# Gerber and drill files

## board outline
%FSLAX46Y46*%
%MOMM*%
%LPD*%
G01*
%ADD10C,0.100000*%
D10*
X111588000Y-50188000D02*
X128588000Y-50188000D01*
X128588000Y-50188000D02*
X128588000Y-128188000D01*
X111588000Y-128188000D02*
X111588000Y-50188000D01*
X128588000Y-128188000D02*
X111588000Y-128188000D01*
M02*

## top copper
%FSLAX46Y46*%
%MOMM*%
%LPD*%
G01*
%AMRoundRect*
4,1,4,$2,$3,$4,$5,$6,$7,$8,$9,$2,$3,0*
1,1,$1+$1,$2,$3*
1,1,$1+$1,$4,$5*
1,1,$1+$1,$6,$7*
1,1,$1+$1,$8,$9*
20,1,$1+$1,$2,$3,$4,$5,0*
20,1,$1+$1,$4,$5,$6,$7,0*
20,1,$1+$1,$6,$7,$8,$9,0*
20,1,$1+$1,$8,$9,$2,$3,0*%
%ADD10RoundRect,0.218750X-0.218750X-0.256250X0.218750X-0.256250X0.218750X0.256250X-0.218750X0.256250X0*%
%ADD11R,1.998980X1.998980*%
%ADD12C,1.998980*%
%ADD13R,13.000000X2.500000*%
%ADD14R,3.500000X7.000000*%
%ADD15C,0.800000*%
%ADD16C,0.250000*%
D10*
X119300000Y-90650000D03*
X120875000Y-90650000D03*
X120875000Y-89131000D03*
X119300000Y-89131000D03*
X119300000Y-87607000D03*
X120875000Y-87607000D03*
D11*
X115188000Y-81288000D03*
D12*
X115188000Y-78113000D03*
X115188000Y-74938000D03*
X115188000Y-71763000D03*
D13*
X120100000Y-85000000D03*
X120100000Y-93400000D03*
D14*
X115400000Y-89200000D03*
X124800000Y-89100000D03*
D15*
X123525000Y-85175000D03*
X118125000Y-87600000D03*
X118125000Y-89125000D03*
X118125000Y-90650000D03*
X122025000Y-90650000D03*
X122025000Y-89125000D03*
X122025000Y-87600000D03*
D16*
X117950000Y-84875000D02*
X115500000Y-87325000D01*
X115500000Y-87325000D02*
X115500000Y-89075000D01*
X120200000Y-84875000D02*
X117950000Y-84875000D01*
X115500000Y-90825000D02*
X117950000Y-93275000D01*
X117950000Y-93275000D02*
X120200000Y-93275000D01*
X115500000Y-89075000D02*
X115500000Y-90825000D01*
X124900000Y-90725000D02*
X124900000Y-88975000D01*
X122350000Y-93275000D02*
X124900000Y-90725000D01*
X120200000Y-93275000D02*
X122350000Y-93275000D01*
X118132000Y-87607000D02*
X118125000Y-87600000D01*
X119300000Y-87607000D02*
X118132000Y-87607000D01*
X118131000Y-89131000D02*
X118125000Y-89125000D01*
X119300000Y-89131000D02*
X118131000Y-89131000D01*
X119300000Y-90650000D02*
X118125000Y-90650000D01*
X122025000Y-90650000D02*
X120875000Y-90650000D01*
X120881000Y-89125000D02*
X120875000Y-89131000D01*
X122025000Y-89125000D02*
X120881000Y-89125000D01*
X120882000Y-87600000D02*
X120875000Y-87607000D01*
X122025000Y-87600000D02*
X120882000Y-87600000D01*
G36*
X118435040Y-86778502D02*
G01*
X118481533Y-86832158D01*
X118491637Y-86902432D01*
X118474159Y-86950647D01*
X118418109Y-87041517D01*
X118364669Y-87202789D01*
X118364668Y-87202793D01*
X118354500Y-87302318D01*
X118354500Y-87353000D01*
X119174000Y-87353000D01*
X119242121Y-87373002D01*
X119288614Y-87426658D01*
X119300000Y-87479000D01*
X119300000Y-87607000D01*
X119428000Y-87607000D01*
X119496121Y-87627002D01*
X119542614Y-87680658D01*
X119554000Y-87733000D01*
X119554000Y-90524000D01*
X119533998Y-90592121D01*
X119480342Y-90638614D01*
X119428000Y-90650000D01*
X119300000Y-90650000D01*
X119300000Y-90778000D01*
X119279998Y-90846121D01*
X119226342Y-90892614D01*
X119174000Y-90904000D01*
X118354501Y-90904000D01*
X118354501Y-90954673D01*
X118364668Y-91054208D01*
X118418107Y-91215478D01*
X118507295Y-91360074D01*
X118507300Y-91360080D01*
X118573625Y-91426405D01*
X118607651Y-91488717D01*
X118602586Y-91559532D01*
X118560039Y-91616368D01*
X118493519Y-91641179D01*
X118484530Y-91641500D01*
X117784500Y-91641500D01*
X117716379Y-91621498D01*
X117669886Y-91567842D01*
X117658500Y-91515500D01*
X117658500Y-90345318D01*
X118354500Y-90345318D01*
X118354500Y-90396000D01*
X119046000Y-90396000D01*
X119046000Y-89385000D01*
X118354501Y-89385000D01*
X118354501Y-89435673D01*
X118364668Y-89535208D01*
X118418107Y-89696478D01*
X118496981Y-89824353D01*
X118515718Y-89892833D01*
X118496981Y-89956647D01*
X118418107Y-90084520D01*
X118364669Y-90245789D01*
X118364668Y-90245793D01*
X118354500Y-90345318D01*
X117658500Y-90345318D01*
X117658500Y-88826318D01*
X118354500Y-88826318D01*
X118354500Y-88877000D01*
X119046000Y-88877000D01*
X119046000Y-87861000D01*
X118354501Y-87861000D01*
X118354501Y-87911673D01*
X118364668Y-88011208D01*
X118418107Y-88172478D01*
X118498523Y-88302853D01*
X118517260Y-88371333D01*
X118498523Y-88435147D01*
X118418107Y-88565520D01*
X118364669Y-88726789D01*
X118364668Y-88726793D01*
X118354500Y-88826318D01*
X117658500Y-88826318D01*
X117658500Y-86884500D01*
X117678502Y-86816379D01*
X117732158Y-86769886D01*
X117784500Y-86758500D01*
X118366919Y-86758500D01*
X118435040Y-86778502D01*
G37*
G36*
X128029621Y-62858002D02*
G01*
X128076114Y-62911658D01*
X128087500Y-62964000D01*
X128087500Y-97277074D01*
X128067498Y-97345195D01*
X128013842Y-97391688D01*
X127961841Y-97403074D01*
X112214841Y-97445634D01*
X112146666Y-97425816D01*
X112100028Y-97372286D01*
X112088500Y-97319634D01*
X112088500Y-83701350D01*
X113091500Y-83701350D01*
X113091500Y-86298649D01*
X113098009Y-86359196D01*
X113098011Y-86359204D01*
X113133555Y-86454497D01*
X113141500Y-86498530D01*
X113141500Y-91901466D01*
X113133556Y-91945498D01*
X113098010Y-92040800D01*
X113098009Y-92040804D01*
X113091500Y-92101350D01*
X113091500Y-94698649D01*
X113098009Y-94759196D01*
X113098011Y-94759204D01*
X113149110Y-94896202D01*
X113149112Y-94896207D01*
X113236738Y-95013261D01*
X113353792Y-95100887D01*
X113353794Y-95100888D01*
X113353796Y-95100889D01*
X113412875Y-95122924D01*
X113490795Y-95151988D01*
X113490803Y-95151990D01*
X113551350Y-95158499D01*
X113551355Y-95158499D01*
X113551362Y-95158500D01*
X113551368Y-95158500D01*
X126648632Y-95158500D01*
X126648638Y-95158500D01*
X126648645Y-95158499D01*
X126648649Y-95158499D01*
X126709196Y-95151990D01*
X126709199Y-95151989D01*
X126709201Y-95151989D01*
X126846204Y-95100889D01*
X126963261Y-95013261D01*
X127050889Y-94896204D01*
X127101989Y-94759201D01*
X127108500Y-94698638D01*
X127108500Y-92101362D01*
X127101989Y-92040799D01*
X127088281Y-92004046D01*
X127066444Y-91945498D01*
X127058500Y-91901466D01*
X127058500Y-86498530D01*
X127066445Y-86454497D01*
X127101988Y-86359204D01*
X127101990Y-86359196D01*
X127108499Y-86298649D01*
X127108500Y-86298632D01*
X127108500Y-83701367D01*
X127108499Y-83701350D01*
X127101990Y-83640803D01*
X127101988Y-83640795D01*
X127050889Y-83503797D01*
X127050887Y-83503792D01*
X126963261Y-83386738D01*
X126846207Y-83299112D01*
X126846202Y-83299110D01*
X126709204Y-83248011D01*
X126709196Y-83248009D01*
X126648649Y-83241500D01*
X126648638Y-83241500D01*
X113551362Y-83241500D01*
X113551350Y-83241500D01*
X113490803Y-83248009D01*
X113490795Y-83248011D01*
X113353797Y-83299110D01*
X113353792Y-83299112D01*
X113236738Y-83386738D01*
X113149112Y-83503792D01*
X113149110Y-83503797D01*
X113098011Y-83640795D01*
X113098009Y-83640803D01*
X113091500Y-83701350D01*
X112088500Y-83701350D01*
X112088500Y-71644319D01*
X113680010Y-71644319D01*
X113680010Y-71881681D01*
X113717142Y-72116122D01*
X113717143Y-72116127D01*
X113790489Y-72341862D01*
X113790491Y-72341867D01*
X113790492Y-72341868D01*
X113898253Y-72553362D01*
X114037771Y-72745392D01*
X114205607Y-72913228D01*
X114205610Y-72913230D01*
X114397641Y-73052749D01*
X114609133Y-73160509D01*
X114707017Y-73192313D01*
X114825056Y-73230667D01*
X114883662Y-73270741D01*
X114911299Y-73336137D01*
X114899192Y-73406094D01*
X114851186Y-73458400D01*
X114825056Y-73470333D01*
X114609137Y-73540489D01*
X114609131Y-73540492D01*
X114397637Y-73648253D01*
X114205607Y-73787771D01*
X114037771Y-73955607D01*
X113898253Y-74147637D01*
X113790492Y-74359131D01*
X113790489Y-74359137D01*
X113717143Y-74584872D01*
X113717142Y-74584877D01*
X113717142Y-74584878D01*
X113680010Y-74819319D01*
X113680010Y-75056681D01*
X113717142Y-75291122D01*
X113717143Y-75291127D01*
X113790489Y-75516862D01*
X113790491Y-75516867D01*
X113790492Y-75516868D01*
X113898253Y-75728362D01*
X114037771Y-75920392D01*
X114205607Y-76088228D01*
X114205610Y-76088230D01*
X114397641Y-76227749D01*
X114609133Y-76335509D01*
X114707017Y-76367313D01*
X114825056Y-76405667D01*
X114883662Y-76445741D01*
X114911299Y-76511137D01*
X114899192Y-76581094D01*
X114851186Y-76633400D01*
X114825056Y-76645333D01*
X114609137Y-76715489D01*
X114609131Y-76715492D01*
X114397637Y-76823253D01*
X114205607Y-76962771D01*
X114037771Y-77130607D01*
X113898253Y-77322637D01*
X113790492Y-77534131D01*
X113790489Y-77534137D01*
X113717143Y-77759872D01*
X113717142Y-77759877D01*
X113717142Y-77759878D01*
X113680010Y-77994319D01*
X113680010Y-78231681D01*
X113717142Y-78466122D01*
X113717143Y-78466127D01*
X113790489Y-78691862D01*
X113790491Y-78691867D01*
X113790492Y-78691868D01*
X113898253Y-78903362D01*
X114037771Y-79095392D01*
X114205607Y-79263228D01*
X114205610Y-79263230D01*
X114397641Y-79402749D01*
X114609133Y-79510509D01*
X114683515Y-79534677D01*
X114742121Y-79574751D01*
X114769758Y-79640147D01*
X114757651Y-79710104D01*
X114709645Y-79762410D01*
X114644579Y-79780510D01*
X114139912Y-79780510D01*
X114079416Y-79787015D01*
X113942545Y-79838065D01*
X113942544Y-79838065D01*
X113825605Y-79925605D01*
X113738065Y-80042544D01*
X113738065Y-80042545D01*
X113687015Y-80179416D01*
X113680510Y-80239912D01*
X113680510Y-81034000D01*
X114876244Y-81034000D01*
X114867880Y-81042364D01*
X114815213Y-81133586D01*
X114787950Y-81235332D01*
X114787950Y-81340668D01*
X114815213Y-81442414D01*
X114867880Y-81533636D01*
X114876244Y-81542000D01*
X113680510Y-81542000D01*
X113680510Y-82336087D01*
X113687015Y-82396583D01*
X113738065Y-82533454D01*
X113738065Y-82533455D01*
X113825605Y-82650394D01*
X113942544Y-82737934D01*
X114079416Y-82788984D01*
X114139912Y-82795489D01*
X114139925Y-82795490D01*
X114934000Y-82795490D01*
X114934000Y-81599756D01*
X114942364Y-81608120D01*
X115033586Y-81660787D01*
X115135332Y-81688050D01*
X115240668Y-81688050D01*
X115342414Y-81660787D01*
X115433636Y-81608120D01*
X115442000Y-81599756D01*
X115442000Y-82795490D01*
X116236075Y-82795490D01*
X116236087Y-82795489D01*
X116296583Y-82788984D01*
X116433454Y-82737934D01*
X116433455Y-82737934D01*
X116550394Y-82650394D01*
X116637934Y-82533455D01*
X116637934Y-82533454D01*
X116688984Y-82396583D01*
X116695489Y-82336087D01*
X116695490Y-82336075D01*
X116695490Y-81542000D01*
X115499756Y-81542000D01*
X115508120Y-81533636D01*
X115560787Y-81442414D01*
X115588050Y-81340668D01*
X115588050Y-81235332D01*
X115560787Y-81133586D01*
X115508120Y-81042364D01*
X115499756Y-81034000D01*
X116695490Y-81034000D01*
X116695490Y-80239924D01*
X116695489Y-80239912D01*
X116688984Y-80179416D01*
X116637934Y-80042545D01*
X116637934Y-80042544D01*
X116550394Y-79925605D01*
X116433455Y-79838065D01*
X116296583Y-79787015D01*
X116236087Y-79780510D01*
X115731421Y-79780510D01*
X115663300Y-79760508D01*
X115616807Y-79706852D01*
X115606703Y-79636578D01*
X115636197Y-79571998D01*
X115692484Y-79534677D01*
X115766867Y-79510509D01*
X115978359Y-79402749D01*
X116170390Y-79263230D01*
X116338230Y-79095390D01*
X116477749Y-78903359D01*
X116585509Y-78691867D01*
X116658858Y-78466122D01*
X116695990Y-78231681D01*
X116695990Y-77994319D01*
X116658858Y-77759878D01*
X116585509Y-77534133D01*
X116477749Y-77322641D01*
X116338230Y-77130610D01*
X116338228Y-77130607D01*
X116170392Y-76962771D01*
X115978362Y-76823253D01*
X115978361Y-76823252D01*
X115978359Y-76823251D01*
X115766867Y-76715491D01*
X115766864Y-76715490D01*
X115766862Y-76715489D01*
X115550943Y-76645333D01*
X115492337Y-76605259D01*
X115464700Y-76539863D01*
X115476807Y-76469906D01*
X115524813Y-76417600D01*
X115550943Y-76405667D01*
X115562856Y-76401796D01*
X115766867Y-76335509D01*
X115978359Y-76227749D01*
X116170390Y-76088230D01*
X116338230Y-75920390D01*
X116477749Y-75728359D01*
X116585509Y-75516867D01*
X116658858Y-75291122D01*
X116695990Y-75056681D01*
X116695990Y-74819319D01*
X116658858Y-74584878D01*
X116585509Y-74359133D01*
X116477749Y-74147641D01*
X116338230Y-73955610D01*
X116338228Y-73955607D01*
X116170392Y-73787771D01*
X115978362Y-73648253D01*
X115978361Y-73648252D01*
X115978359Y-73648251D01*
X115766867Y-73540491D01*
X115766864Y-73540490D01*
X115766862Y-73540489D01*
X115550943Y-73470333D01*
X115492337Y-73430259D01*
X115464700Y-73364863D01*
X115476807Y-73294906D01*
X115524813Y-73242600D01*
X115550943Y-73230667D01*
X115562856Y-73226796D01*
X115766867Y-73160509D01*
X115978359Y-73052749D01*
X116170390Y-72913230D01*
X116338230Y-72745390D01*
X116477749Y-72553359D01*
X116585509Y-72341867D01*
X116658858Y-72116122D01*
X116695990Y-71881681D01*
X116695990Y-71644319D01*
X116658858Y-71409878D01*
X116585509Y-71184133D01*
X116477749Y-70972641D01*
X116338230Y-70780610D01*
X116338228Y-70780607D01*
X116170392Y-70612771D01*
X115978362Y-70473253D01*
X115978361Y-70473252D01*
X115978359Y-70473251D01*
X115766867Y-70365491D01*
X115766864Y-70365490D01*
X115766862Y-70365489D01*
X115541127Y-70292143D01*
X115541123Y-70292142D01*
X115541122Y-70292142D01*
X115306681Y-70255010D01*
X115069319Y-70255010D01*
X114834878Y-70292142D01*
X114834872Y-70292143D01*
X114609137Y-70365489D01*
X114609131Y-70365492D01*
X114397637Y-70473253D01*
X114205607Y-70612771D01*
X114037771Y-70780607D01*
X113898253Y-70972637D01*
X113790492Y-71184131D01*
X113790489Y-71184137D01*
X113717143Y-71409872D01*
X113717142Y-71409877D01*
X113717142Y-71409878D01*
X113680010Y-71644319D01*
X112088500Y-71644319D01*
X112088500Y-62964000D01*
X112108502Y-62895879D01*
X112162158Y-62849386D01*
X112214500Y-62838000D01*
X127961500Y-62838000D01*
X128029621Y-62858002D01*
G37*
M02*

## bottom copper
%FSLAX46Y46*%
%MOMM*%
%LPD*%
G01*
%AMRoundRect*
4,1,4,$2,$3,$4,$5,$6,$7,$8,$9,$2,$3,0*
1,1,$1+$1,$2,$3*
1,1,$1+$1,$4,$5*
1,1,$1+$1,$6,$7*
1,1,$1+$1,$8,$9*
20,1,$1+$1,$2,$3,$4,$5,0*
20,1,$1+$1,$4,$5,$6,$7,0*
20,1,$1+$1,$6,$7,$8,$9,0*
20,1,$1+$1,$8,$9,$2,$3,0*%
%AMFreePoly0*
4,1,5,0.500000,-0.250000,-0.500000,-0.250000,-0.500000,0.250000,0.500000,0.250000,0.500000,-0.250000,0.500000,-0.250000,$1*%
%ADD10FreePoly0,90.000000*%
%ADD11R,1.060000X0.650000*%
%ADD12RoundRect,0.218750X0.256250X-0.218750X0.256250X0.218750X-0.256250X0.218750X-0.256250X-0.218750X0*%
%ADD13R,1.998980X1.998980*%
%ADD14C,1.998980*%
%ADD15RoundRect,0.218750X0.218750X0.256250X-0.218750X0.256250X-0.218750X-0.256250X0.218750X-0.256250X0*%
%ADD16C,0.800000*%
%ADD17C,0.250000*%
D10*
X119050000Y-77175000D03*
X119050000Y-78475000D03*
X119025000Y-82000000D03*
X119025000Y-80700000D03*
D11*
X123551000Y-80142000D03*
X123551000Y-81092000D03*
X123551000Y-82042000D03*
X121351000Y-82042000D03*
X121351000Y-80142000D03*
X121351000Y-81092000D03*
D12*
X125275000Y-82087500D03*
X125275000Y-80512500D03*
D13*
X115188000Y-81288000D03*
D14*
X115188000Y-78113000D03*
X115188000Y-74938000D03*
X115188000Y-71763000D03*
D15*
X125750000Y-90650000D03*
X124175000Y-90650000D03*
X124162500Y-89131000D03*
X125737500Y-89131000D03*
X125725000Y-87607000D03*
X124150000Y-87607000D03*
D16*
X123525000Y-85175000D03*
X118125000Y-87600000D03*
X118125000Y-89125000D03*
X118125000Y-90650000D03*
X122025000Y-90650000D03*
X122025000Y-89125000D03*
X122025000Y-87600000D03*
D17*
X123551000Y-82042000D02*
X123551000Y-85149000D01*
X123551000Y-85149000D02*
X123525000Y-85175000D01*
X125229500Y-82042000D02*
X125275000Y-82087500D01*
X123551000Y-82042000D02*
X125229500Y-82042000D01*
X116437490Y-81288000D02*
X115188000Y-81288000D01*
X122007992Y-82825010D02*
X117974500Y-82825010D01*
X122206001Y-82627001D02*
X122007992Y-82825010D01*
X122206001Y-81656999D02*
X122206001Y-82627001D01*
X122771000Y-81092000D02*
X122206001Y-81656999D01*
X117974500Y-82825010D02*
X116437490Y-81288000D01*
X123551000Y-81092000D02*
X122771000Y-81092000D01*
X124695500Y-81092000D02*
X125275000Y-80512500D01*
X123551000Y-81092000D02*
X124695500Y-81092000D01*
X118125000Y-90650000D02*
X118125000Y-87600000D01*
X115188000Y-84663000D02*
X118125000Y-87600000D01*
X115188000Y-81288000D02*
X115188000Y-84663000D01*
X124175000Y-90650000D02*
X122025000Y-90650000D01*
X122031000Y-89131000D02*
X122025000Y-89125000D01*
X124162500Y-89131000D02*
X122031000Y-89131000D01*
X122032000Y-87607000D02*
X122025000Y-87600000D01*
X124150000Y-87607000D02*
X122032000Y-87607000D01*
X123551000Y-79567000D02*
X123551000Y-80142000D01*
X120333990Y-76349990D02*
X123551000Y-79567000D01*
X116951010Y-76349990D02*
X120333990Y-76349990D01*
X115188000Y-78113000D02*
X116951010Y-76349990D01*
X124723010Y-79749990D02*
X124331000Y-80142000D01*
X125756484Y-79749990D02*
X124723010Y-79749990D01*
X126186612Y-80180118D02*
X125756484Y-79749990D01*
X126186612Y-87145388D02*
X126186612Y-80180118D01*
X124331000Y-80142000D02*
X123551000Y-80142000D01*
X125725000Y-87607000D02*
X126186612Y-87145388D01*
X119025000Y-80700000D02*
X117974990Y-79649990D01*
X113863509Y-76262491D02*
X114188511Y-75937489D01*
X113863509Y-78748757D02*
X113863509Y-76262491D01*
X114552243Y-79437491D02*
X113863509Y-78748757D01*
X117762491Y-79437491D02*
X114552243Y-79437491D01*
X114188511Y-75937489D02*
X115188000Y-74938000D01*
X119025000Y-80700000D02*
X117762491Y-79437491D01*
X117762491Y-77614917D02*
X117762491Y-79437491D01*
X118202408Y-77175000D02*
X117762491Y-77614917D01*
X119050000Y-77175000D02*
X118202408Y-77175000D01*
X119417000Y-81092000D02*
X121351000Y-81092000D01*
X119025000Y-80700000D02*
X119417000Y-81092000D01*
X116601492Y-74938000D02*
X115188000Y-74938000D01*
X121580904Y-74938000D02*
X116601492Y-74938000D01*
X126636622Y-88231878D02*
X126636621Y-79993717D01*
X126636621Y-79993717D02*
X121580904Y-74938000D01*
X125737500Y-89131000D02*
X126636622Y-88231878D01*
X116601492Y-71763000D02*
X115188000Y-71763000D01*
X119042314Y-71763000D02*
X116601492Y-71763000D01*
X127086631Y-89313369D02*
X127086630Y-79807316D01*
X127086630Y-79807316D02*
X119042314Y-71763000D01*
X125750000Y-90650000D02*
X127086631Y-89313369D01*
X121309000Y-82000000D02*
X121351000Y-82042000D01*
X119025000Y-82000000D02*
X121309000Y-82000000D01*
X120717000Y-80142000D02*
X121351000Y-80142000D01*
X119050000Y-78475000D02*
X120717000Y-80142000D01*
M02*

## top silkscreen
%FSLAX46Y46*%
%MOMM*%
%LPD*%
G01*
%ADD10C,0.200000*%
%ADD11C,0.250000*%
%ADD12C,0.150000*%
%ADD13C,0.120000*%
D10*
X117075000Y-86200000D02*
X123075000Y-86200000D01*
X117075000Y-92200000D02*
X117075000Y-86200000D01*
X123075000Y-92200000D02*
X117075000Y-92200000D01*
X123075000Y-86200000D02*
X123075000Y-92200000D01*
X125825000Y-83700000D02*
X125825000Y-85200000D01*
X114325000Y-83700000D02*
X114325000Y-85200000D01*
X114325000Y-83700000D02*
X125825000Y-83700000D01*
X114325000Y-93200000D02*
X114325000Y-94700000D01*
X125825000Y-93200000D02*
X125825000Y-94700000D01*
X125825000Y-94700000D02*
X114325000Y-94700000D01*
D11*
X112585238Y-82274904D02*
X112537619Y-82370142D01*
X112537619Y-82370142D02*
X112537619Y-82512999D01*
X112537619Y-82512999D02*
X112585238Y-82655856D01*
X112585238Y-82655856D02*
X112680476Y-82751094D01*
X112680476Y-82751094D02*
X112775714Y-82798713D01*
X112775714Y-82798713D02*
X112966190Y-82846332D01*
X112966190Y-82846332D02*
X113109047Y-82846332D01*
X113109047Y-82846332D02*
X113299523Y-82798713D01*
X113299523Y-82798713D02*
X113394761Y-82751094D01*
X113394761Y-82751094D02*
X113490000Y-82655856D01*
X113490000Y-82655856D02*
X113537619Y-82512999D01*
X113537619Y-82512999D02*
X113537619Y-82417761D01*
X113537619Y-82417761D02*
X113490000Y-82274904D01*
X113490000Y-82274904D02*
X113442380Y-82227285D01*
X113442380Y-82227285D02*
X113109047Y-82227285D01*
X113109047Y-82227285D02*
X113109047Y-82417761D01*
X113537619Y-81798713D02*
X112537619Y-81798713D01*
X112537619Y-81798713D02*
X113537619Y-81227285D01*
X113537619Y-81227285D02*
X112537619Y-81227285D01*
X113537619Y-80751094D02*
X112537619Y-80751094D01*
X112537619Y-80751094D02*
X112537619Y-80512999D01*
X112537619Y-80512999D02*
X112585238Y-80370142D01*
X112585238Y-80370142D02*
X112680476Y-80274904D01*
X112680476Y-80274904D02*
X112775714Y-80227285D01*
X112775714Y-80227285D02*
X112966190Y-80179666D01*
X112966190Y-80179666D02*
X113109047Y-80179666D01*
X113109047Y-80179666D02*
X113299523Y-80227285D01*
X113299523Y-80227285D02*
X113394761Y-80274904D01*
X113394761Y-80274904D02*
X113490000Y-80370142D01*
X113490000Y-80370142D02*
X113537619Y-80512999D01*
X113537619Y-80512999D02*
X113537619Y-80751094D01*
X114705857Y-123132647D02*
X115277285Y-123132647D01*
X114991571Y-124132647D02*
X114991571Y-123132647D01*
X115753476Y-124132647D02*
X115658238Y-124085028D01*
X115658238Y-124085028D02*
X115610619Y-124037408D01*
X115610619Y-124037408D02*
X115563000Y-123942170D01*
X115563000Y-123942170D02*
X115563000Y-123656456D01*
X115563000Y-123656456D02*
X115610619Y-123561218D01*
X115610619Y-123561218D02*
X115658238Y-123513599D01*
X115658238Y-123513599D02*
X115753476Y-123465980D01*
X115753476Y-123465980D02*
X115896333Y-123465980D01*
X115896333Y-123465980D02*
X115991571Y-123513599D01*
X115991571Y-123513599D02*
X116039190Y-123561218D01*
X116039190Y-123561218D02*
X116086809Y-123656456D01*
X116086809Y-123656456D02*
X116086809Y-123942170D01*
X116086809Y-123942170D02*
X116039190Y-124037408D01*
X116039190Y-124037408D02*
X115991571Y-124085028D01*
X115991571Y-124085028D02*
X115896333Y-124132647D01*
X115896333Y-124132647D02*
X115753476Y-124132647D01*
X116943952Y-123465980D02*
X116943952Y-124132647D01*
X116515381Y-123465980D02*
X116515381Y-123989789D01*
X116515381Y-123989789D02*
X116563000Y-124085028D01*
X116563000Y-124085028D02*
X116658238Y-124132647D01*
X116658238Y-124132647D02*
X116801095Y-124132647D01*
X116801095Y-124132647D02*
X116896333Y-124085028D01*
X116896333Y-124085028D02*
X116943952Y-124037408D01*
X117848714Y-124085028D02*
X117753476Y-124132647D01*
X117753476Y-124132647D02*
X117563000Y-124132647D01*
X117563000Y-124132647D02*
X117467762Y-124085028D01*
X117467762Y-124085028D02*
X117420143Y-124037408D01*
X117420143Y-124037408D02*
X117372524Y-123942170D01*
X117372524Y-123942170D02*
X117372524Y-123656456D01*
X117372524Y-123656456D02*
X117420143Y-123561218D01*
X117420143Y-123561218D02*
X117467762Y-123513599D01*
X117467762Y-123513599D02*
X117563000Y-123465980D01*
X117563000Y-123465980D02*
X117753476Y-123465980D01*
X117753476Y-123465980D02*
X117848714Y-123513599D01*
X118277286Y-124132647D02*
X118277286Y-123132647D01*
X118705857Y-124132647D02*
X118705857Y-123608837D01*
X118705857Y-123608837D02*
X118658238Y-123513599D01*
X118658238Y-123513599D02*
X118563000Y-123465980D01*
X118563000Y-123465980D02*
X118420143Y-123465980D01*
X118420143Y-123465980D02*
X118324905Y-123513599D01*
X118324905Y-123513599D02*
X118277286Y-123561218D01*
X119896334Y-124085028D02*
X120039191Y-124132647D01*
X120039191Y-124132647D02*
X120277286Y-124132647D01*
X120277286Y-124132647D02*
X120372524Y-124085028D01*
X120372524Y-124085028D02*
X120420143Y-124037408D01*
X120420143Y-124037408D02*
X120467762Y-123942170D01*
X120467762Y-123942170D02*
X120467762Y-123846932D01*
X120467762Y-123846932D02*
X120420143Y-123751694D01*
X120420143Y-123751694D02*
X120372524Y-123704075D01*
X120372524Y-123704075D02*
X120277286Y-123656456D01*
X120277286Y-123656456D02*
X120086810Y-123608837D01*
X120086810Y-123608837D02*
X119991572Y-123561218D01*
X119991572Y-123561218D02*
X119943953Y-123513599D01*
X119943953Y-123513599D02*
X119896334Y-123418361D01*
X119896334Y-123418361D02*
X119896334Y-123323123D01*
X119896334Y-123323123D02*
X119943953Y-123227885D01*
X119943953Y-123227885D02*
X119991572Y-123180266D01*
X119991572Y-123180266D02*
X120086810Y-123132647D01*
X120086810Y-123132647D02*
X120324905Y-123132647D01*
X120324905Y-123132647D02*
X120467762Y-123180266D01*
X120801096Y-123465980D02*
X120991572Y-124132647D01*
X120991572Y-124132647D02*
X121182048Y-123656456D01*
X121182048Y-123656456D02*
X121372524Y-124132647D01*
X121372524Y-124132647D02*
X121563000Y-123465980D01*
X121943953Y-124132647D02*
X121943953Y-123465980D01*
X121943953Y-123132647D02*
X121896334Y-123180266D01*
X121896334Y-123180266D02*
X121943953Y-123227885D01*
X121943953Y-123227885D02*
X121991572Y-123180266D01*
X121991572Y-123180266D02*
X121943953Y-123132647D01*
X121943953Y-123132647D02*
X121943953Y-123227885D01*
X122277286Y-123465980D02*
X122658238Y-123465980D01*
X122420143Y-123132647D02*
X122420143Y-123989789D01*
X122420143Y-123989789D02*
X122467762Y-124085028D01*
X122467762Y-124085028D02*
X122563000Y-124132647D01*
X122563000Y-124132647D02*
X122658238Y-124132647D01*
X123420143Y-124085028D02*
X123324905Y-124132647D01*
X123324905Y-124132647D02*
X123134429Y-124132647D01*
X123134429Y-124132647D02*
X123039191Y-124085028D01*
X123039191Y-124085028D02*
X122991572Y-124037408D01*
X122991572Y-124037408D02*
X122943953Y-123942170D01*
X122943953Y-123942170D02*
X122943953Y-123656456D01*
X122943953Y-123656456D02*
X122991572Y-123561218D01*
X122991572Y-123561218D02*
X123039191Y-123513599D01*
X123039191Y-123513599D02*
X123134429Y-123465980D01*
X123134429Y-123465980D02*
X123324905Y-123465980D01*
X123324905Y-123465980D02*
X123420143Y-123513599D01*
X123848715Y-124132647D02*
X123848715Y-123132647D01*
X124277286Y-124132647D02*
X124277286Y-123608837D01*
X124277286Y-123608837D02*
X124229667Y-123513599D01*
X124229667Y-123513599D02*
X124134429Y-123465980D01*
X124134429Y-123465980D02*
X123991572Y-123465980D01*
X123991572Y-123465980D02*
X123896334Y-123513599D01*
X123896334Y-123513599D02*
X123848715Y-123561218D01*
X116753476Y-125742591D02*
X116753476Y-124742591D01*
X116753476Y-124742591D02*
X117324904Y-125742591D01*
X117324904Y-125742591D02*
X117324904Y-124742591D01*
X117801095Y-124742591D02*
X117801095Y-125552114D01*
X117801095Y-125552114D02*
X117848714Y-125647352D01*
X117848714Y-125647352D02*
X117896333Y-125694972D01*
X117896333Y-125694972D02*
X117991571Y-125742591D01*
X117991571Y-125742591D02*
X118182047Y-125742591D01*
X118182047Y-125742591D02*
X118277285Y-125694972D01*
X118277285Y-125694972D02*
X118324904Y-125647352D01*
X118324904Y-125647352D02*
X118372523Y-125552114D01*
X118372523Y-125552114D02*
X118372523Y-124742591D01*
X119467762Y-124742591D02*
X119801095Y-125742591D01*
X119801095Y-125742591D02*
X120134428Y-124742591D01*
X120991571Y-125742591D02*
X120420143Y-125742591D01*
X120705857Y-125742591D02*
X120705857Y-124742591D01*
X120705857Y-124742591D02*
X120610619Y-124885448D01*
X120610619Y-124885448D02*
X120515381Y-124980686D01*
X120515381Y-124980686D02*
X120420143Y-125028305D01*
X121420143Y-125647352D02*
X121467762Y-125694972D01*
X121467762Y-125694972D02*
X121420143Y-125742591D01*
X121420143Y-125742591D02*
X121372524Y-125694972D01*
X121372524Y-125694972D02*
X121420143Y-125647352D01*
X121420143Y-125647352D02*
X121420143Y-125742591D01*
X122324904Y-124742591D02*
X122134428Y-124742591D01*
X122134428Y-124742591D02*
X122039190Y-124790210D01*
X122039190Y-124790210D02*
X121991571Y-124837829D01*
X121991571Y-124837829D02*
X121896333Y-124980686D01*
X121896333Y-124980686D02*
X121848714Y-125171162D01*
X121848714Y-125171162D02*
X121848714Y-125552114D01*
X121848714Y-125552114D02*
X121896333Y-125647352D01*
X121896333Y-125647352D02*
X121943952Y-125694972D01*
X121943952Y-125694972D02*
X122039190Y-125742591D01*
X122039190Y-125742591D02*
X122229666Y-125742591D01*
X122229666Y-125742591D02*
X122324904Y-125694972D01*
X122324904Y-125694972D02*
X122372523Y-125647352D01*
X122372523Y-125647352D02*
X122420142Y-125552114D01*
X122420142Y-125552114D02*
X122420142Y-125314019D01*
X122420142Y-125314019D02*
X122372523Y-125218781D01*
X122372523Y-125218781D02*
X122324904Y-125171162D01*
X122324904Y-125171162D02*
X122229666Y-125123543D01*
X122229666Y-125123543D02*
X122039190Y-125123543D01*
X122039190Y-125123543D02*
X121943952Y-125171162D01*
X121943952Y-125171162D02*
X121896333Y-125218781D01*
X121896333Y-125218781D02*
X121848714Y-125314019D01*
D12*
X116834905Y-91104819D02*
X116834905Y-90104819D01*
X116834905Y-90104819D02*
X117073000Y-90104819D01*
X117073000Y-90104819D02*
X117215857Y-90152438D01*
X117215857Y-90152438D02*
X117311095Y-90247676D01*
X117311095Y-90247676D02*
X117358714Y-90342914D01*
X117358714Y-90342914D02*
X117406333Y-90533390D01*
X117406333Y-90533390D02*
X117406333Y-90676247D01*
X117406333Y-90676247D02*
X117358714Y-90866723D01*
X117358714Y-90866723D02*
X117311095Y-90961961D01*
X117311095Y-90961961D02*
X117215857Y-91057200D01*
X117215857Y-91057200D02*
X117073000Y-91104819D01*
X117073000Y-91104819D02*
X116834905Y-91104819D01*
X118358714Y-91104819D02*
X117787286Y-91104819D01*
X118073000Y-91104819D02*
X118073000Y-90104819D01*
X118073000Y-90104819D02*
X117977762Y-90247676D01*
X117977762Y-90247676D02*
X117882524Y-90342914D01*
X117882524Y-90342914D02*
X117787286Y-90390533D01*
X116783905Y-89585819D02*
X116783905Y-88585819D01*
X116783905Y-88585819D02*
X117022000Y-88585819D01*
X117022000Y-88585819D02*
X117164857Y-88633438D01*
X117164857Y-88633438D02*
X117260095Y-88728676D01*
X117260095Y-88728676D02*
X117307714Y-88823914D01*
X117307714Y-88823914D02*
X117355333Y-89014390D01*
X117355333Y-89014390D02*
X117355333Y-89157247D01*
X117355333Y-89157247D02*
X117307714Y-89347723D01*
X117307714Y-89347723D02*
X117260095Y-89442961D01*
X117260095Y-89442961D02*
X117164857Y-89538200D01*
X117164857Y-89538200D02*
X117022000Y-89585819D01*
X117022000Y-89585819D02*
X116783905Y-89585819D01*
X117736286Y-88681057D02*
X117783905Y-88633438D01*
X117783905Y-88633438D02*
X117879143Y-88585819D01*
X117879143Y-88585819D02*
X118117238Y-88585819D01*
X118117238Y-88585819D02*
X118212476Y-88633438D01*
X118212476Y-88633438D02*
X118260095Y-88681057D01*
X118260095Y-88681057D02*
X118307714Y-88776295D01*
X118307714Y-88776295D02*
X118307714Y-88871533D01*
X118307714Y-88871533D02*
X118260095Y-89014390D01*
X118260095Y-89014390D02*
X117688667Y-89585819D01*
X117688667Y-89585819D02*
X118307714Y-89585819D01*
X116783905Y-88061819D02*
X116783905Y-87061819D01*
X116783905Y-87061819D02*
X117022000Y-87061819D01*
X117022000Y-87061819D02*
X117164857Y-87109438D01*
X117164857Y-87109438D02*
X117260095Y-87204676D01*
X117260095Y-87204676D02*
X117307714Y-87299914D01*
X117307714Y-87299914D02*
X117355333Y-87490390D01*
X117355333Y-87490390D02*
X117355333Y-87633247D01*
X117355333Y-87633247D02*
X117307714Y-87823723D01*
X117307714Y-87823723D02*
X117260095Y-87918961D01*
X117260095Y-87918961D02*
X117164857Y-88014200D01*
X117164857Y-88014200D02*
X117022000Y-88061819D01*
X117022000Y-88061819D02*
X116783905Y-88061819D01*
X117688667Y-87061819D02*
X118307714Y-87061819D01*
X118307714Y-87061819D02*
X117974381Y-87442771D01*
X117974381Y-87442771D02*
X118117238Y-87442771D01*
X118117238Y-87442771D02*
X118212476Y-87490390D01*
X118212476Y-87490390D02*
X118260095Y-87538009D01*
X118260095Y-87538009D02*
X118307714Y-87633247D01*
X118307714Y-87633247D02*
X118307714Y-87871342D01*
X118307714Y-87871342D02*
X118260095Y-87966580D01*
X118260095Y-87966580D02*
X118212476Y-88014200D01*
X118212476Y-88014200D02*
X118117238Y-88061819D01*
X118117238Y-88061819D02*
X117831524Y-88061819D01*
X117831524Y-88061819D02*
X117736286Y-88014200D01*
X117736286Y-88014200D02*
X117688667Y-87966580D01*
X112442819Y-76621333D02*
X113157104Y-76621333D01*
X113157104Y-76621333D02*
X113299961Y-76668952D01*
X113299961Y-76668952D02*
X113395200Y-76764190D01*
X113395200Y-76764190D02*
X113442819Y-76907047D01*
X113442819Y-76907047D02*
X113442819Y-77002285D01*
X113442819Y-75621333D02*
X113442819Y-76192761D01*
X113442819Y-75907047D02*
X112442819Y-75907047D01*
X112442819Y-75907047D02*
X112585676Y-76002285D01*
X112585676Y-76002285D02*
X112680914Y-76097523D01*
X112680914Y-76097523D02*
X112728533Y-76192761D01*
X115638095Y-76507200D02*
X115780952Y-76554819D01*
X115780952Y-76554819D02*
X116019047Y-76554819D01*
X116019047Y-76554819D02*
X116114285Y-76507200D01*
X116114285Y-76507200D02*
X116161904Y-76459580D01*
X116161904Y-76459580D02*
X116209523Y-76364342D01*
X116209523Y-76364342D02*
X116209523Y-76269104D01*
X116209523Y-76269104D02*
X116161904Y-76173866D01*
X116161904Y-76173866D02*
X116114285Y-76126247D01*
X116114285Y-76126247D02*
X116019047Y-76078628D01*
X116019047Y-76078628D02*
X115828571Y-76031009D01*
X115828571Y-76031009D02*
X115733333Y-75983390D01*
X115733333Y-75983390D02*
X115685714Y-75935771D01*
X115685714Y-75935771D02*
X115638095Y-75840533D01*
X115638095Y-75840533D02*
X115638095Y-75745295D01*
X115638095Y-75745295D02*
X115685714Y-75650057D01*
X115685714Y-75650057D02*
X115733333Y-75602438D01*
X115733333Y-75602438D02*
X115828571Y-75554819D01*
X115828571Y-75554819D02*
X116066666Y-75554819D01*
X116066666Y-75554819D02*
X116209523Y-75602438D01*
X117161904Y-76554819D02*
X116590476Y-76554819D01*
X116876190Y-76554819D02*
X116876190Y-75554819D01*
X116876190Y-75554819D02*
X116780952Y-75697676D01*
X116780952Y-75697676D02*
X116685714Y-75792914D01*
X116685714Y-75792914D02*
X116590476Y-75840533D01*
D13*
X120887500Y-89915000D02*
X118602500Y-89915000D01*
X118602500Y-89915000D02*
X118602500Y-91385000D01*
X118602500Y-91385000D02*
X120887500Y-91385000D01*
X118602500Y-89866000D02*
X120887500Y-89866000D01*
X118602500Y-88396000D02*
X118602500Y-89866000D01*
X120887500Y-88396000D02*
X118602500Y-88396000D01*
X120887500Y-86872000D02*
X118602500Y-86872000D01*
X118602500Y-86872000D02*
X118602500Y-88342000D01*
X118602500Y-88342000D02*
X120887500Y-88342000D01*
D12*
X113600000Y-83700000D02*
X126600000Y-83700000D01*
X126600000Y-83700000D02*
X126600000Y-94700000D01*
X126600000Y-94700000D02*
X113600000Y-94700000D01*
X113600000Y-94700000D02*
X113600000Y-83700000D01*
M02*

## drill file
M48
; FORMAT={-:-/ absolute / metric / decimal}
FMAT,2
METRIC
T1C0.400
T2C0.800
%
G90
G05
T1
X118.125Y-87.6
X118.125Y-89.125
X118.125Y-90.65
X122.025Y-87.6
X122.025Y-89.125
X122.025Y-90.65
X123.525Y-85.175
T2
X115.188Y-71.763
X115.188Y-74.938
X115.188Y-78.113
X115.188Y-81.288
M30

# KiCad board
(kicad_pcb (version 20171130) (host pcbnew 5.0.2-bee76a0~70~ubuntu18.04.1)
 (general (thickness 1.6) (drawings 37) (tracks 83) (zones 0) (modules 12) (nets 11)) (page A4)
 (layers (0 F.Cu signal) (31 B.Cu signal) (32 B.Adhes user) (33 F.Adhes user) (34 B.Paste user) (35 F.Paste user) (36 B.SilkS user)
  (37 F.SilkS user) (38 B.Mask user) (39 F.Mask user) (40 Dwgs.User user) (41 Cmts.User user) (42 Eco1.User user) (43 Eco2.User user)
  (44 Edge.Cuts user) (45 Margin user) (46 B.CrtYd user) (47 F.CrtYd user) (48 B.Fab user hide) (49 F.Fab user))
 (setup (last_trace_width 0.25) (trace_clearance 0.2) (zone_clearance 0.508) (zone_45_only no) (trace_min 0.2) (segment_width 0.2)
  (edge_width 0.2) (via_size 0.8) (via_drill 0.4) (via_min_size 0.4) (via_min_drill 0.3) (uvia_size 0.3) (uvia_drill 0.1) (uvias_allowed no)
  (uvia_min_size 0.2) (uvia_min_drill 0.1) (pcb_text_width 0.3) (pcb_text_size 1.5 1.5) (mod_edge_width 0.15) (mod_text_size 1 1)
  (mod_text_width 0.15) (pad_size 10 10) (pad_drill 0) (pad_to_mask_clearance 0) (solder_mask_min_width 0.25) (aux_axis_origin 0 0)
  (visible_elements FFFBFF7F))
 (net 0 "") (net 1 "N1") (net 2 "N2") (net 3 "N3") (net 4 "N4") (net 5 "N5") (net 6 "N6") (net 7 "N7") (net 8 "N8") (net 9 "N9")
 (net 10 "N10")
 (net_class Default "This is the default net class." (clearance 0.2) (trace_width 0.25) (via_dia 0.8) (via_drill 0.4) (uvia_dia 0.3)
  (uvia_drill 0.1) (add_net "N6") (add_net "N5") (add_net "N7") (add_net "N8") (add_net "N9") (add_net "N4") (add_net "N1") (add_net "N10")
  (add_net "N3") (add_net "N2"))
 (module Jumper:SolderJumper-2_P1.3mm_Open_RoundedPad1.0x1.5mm (layer B.Cu) (at 119.05 77.825 90)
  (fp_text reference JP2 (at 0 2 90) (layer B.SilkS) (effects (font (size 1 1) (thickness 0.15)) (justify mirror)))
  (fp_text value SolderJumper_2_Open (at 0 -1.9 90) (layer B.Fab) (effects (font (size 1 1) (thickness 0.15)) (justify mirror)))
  (pad 2 smd custom (at 0.65 0 90) (size 1 0.5) (layers B.Cu B.Mask) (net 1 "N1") (zone_connect 0)
   (options (clearance outline) (anchor rect)) (primitives))
  (pad 1 smd custom (at -0.65 0 90) (size 1 0.5) (layers B.Cu B.Mask) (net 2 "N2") (zone_connect 0)
   (options (clearance outline) (anchor rect)) (primitives)))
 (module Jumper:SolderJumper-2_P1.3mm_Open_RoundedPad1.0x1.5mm (layer B.Cu) (at 119.025 81.35 90)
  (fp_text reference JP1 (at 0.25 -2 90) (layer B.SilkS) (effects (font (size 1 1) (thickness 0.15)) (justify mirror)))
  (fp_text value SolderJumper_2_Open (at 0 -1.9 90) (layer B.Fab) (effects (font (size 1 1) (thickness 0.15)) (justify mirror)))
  (pad 1 smd custom (at -0.65 0 90) (size 1 0.5) (layers B.Cu B.Mask) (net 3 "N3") (zone_connect 0)
   (options (clearance outline) (anchor rect)) (primitives))
  (pad 2 smd custom (at 0.65 0 90) (size 1 0.5) (layers B.Cu B.Mask) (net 1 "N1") (zone_connect 0)
   (options (clearance outline) (anchor rect)) (primitives)))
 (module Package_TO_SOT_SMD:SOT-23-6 (layer B.Cu) (at 122.451 81.092 180)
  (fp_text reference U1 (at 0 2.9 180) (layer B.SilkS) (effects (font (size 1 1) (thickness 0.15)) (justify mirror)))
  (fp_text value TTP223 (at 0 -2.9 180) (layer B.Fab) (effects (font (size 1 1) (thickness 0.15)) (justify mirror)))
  (pad 1 smd rect (at -1.1 0.95 180) (size 1.06 0.65) (layers B.Cu B.Paste B.Mask) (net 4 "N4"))
  (pad 2 smd rect (at -1.1 0 180) (size 1.06 0.65) (layers B.Cu B.Paste B.Mask) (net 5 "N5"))
  (pad 3 smd rect (at -1.1 -0.95 180) (size 1.06 0.65) (layers B.Cu B.Paste B.Mask) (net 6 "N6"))
  (pad 4 smd rect (at 1.1 -0.95 180) (size 1.06 0.65) (layers B.Cu B.Paste B.Mask) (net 3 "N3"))
  (pad 6 smd rect (at 1.1 0.95 180) (size 1.06 0.65) (layers B.Cu B.Paste B.Mask) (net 2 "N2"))
  (pad 5 smd rect (at 1.1 0 180) (size 1.06 0.65) (layers B.Cu B.Paste B.Mask) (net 1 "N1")))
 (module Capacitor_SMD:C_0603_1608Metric (layer B.Cu) (at 125.275 81.3 90)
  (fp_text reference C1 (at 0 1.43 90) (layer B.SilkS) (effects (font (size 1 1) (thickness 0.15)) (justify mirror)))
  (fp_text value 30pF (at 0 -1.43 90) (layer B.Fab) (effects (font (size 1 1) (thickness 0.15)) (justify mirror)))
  (pad 1 smd roundrect (at -0.7875 0 90) (size 0.875 0.95) (layers B.Cu B.Paste B.Mask) (roundrect_rratio 0.25) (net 6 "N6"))
  (pad 2 smd roundrect (at 0.7875 0 90) (size 0.875 0.95) (layers B.Cu B.Paste B.Mask) (roundrect_rratio 0.25) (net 5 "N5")))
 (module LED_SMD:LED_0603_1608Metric (layer F.Cu) (at 120.0875 90.65)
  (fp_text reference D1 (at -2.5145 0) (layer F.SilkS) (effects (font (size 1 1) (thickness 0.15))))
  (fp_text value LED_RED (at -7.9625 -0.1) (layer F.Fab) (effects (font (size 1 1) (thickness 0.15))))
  (fp_line (start 0.8 -0.735) (end -1.485 -0.735) (layer F.SilkS) (width 0.12))
  (fp_line (start -1.485 -0.735) (end -1.485 0.735) (layer F.SilkS) (width 0.12))
  (fp_line (start -1.485 0.735) (end 0.8 0.735) (layer F.SilkS) (width 0.12))
  (pad 1 smd roundrect (at -0.7875 0) (size 0.875 0.95) (layers F.Cu F.Paste F.Mask) (roundrect_rratio 0.25) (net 5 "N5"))
  (pad 2 smd roundrect (at 0.7875 0) (size 0.875 0.95) (layers F.Cu F.Paste F.Mask) (roundrect_rratio 0.25) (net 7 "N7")))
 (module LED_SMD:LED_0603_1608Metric (layer F.Cu) (at 120.0875 89.131)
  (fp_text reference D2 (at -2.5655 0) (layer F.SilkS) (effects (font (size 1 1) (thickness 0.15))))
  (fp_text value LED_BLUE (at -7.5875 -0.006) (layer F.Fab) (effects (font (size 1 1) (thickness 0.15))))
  (fp_line (start -1.485 0.735) (end 0.8 0.735) (layer F.SilkS) (width 0.12))
  (fp_line (start -1.485 -0.735) (end -1.485 0.735) (layer F.SilkS) (width 0.12))
  (fp_line (start 0.8 -0.735) (end -1.485 -0.735) (layer F.SilkS) (width 0.12))
  (pad 2 smd roundrect (at 0.7875 0) (size 0.875 0.95) (layers F.Cu F.Paste F.Mask) (roundrect_rratio 0.25) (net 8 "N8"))
  (pad 1 smd roundrect (at -0.7875 0) (size 0.875 0.95) (layers F.Cu F.Paste F.Mask) (roundrect_rratio 0.25) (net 5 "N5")))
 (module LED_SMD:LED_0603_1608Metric (layer F.Cu) (at 120.0875 87.607)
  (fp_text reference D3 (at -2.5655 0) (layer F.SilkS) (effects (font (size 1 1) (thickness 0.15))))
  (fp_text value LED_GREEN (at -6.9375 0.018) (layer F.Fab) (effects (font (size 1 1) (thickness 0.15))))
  (fp_line (start 0.8 -0.735) (end -1.485 -0.735) (layer F.SilkS) (width 0.12))
  (fp_line (start -1.485 -0.735) (end -1.485 0.735) (layer F.SilkS) (width 0.12))
  (fp_line (start -1.485 0.735) (end 0.8 0.735) (layer F.SilkS) (width 0.12))
  (pad 1 smd roundrect (at -0.7875 0) (size 0.875 0.95) (layers F.Cu F.Paste F.Mask) (roundrect_rratio 0.25) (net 5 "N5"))
  (pad 2 smd roundrect (at 0.7875 0) (size 0.875 0.95) (layers F.Cu F.Paste F.Mask) (roundrect_rratio 0.25) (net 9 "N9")))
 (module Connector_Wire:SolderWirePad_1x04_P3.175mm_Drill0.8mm (layer F.Cu) (at 115.188 81.288 90)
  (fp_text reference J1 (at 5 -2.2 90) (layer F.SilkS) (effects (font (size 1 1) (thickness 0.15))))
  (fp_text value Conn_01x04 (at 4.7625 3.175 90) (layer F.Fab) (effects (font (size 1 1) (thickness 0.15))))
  (pad 1 thru_hole rect (at 0 0 90) (size 1.99898 1.99898) (drill 0.8001) (layers *.Cu *.Mask) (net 5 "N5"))
  (pad 2 thru_hole circle (at 3.175 0 90) (size 1.99898 1.99898) (drill 0.8001) (layers *.Cu *.Mask) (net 4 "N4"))
  (pad 3 thru_hole circle (at 6.35 0 90) (size 1.99898 1.99898) (drill 0.8001) (layers *.Cu *.Mask) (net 1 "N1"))
  (pad 4 thru_hole circle (at 9.525 0 90) (size 1.99898 1.99898) (drill 0.8001) (layers *.Cu *.Mask) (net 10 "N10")))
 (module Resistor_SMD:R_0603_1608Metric (layer B.Cu) (at 124.9625 90.65 180)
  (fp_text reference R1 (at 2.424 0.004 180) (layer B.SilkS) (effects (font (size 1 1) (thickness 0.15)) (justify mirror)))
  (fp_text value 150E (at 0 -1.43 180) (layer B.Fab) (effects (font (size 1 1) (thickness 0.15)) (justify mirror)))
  (pad 1 smd roundrect (at -0.7875 0 180) (size 0.875 0.95) (layers B.Cu B.Paste B.Mask) (roundrect_rratio 0.25) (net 10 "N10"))
  (pad 2 smd roundrect (at 0.7875 0 180) (size 0.875 0.95) (layers B.Cu B.Paste B.Mask) (roundrect_rratio 0.25) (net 7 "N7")))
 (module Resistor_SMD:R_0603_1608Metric (layer B.Cu) (at 124.95 89.131 180)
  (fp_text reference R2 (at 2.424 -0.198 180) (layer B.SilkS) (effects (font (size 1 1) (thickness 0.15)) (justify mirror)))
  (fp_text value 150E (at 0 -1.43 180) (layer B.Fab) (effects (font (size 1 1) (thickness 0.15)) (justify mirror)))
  (pad 2 smd roundrect (at 0.7875 0 180) (size 0.875 0.95) (layers B.Cu B.Paste B.Mask) (roundrect_rratio 0.25) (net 8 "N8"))
  (pad 1 smd roundrect (at -0.7875 0 180) (size 0.875 0.95) (layers B.Cu B.Paste B.Mask) (roundrect_rratio 0.25) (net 1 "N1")))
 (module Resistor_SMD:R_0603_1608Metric (layer B.Cu) (at 124.9375 87.607 180)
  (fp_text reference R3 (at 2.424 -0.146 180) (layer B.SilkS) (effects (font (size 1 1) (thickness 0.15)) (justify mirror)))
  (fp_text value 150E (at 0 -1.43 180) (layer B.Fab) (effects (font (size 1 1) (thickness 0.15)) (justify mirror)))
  (pad 1 smd roundrect (at -0.7875 0 180) (size 0.875 0.95) (layers B.Cu B.Paste B.Mask) (roundrect_rratio 0.25) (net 4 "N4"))
  (pad 2 smd roundrect (at 0.7875 0 180) (size 0.875 0.95) (layers B.Cu B.Paste B.Mask) (roundrect_rratio 0.25) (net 9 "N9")))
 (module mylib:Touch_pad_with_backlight (layer F.Cu) (at 113.6 83.7)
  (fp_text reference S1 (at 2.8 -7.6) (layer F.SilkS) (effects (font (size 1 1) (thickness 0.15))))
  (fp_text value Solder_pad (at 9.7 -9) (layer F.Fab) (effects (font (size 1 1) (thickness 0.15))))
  (fp_line (start 0 0) (end 13 0) (layer F.SilkS) (width 0.15))
  (fp_line (start 13 0) (end 13 11) (layer F.SilkS) (width 0.15))
  (fp_line (start 13 11) (end 0 11) (layer F.SilkS) (width 0.15))
  (fp_line (start 0 11) (end 0 0) (layer F.SilkS) (width 0.15))
  (pad 1 smd rect (at 6.5 1.3) (size 13 2.5) (layers F.Cu F.Paste F.Mask) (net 6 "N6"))
  (pad 1 smd rect (at 6.5 9.7) (size 13 2.5) (layers F.Cu F.Paste F.Mask) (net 6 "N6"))
  (pad 1 smd rect (at 1.8 5.5) (size 3.5 7) (layers F.Cu F.Paste F.Mask) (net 6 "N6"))
  (pad 1 smd rect (at 11.2 5.4) (size 3.5 7) (layers F.Cu F.Paste F.Mask) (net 6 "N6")))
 (gr_line (start 117.075 86.2) (end 123.075 86.2) (layer F.SilkS) (width 0.2))
 (gr_line (start 117.075 92.2) (end 117.075 86.2) (layer F.SilkS) (width 0.2))
 (gr_line (start 123.075 92.2) (end 117.075 92.2) (layer F.SilkS) (width 0.2))
 (gr_line (start 123.075 86.2) (end 123.075 92.2) (layer F.SilkS) (width 0.2))
 (gr_line (start 125.825 83.7) (end 125.825 85.2) (layer F.SilkS) (width 0.2))
 (gr_line (start 114.325 83.7) (end 114.325 85.2) (layer F.SilkS) (width 0.2))
 (gr_line (start 114.325 83.7) (end 125.825 83.7) (layer F.SilkS) (width 0.2))
 (gr_line (start 114.325 93.2) (end 114.325 94.7) (layer F.SilkS) (width 0.2))
 (gr_line (start 125.825 93.2) (end 125.825 94.7) (layer F.SilkS) (width 0.2))
 (gr_line (start 125.825 94.7) (end 114.325 94.7) (layer F.SilkS) (width 0.2))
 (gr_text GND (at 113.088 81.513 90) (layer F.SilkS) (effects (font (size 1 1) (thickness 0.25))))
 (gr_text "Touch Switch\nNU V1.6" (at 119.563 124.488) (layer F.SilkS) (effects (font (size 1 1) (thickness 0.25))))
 (gr_line (start 111.588 50.188) (end 128.588 50.188) (layer Edge.Cuts) (width 0.1))
 (gr_line (start 128.588 50.188) (end 128.588 128.188) (layer Edge.Cuts) (width 0.1))
 (gr_line (start 111.588 128.188) (end 111.588 50.188) (layer Edge.Cuts) (width 0.1))
 (gr_line (start 128.588 128.188) (end 111.588 128.188) (layer Edge.Cuts) (width 0.1))
 (via (at 123.525 85.175) (size 0.8) (drill 0.4) (layers F.Cu B.Cu) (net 6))
 (segment (start 123.551 82.042) (end 123.551 85.149) (width 0.25) (layer B.Cu) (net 6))
 (segment (start 123.551 85.149) (end 123.525 85.175) (width 0.25) (layer B.Cu) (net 6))
 (segment (start 125.2295 82.042) (end 125.275 82.0875) (width 0.25) (layer B.Cu) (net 6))
 (segment (start 123.551 82.042) (end 125.2295 82.042) (width 0.25) (layer B.Cu) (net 6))
 (segment (start 117.95 84.875) (end 115.5 87.325) (width 0.25) (layer F.Cu) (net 6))
 (segment (start 115.5 87.325) (end 115.5 89.075) (width 0.25) (layer F.Cu) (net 6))
 (segment (start 120.2 84.875) (end 117.95 84.875) (width 0.25) (layer F.Cu) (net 6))
 (segment (start 115.5 90.825) (end 117.95 93.275) (width 0.25) (layer F.Cu) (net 6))
 (segment (start 117.95 93.275) (end 120.2 93.275) (width 0.25) (layer F.Cu) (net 6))
 (segment (start 115.5 89.075) (end 115.5 90.825) (width 0.25) (layer F.Cu) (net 6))
 (segment (start 124.9 90.725) (end 124.9 88.975) (width 0.25) (layer F.Cu) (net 6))
 (segment (start 122.35 93.275) (end 124.9 90.725) (width 0.25) (layer F.Cu) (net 6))
 (segment (start 120.2 93.275) (end 122.35 93.275) (width 0.25) (layer F.Cu) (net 6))
 (via (at 118.125 87.6) (size 0.8) (drill 0.4) (layers F.Cu B.Cu) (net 5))
 (via (at 118.125 89.125) (size 0.8) (drill 0.4) (layers F.Cu B.Cu) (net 5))
 (via (at 118.125 90.65) (size 0.8) (drill 0.4) (layers F.Cu B.Cu) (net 5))
 (segment (start 116.43749 81.288) (end 115.188 81.288) (width 0.25) (layer B.Cu) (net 5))
 (segment (start 122.007992 82.82501) (end 117.9745 82.82501) (width 0.25) (layer B.Cu) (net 5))
 (segment (start 122.206001 82.627001) (end 122.007992 82.82501) (width 0.25) (layer B.Cu) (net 5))
 (segment (start 122.206001 81.656999) (end 122.206001 82.627001) (width 0.25) (layer B.Cu) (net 5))
 (segment (start 122.771 81.092) (end 122.206001 81.656999) (width 0.25) (layer B.Cu) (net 5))
 (segment (start 117.9745 82.82501) (end 116.43749 81.288) (width 0.25) (layer B.Cu) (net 5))
 (segment (start 123.551 81.092) (end 122.771 81.092) (width 0.25) (layer B.Cu) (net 5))
 (segment (start 124.6955 81.092) (end 125.275 80.5125) (width 0.25) (layer B.Cu) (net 5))
 (segment (start 123.551 81.092) (end 124.6955 81.092) (width 0.25) (layer B.Cu) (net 5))
 (segment (start 118.132 87.607) (end 118.125 87.6) (width 0.25) (layer F.Cu) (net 5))
 (segment (start 119.3 87.607) (end 118.132 87.607) (width 0.25) (layer F.Cu) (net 5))
 (segment (start 118.131 89.131) (end 118.125 89.125) (width 0.25) (layer F.Cu) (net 5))
 (segment (start 119.3 89.131) (end 118.131 89.131) (width 0.25) (layer F.Cu) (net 5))
 (segment (start 119.3 90.65) (end 118.125 90.65) (width 0.25) (layer F.Cu) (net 5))
 (segment (start 118.125 90.65) (end 118.125 87.6) (width 0.25) (layer B.Cu) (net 5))
 (segment (start 115.188 84.663) (end 118.125 87.6) (width 0.25) (layer B.Cu) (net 5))
 (segment (start 115.188 81.288) (end 115.188 84.663) (width 0.25) (layer B.Cu) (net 5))
 (via (at 122.025 90.65) (size 0.8) (drill 0.4) (layers F.Cu B.Cu) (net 7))
 (segment (start 124.175 90.65) (end 122.025 90.65) (width 0.25) (layer B.Cu) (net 7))
 (segment (start 122.025 90.65) (end 120.875 90.65) (width 0.25) (layer F.Cu) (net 7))
 (via (at 122.025 89.125) (size 0.8) (drill 0.4) (layers F.Cu B.Cu) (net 8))
 (segment (start 122.031 89.131) (end 122.025 89.125) (width 0.25) (layer B.Cu) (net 8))
 (segment (start 124.1625 89.131) (end 122.031 89.131) (width 0.25) (layer B.Cu) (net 8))
 (segment (start 120.881 89.125) (end 120.875 89.131) (width 0.25) (layer F.Cu) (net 8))
 (segment (start 122.025 89.125) (end 120.881 89.125) (width 0.25) (layer F.Cu) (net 8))
 (via (at 122.025 87.6) (size 0.8) (drill 0.4) (layers F.Cu B.Cu) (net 9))
 (segment (start 122.032 87.607) (end 122.025 87.6) (width 0.25) (layer B.Cu) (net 9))
 (segment (start 124.15 87.607) (end 122.032 87.607) (width 0.25) (layer B.Cu) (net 9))
 (segment (start 120.882 87.6) (end 120.875 87.607) (width 0.25) (layer F.Cu) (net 9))
 (segment (start 122.025 87.6) (end 120.882 87.6) (width 0.25) (layer F.Cu) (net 9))
 (segment (start 123.551 79.567) (end 123.551 80.142) (width 0.25) (layer B.Cu) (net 4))
 (segment (start 120.33399 76.34999) (end 123.551 79.567) (width 0.25) (layer B.Cu) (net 4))
 (segment (start 116.95101 76.34999) (end 120.33399 76.34999) (width 0.25) (layer B.Cu) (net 4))
 (segment (start 115.188 78.113) (end 116.95101 76.34999) (width 0.25) (layer B.Cu) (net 4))
 (segment (start 124.72301 79.74999) (end 124.331 80.142) (width 0.25) (layer B.Cu) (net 4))
 (segment (start 125.756484 79.74999) (end 124.72301 79.74999) (width 0.25) (layer B.Cu) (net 4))
 (segment (start 126.186612 80.180118) (end 125.756484 79.74999) (width 0.25) (layer B.Cu) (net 4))
 (segment (start 126.186612 87.145388) (end 126.186612 80.180118) (width 0.25) (layer B.Cu) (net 4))
 (segment (start 124.331 80.142) (end 123.551 80.142) (width 0.25) (layer B.Cu) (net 4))
 (segment (start 125.725 87.607) (end 126.186612 87.145388) (width 0.25) (layer B.Cu) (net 4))
 (segment (start 119.025 80.7) (end 117.97499 79.64999) (width 0.25) (layer B.Cu) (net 1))
 (segment (start 113.863509 76.262491) (end 114.188511 75.937489) (width 0.25) (layer B.Cu) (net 1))
 (segment (start 113.863509 78.748757) (end 113.863509 76.262491) (width 0.25) (layer B.Cu) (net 1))
 (segment (start 114.552243 79.437491) (end 113.863509 78.748757) (width 0.25) (layer B.Cu) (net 1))
 (segment (start 117.762491 79.437491) (end 114.552243 79.437491) (width 0.25) (layer B.Cu) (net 1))
 (segment (start 114.188511 75.937489) (end 115.188 74.938) (width 0.25) (layer B.Cu) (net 1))
 (segment (start 119.025 80.7) (end 117.762491 79.437491) (width 0.25) (layer B.Cu) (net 1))
 (segment (start 117.762491 77.614917) (end 117.762491 79.437491) (width 0.25) (layer B.Cu) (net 1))
 (segment (start 118.202408 77.175) (end 117.762491 77.614917) (width 0.25) (layer B.Cu) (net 1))
 (segment (start 119.05 77.175) (end 118.202408 77.175) (width 0.25) (layer B.Cu) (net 1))
 (segment (start 119.417 81.092) (end 121.351 81.092) (width 0.25) (layer B.Cu) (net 1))
 (segment (start 119.025 80.7) (end 119.417 81.092) (width 0.25) (layer B.Cu) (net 1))
 (segment (start 116.601492 74.938) (end 115.188 74.938) (width 0.25) (layer B.Cu) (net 1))
 (segment (start 121.580904 74.938) (end 116.601492 74.938) (width 0.25) (layer B.Cu) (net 1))
 (segment (start 126.636622 88.231878) (end 126.636621 79.993717) (width 0.25) (layer B.Cu) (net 1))
 (segment (start 126.636621 79.993717) (end 121.580904 74.938) (width 0.25) (layer B.Cu) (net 1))
 (segment (start 125.7375 89.131) (end 126.636622 88.231878) (width 0.25) (layer B.Cu) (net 1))
 (segment (start 116.601492 71.763) (end 115.188 71.763) (width 0.25) (layer B.Cu) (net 10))
 (segment (start 119.042314 71.763) (end 116.601492 71.763) (width 0.25) (layer B.Cu) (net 10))
 (segment (start 127.086631 89.313369) (end 127.08663 79.807316) (width 0.25) (layer B.Cu) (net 10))
 (segment (start 127.08663 79.807316) (end 119.042314 71.763) (width 0.25) (layer B.Cu) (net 10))
 (segment (start 125.75 90.65) (end 127.086631 89.313369) (width 0.25) (layer B.Cu) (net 10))
 (segment (start 121.309 82) (end 121.351 82.042) (width 0.25) (layer B.Cu) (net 3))
 (segment (start 119.025 82) (end 121.309 82) (width 0.25) (layer B.Cu) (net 3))
 (segment (start 120.717 80.142) (end 121.351 80.142) (width 0.25) (layer B.Cu) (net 2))
 (segment (start 119.05 78.475) (end 120.717 80.142) (width 0.25) (layer B.Cu) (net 2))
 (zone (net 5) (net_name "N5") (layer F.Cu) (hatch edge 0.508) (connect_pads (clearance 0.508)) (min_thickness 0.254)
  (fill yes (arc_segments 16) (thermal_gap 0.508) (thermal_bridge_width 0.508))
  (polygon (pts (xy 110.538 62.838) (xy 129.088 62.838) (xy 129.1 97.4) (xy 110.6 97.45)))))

